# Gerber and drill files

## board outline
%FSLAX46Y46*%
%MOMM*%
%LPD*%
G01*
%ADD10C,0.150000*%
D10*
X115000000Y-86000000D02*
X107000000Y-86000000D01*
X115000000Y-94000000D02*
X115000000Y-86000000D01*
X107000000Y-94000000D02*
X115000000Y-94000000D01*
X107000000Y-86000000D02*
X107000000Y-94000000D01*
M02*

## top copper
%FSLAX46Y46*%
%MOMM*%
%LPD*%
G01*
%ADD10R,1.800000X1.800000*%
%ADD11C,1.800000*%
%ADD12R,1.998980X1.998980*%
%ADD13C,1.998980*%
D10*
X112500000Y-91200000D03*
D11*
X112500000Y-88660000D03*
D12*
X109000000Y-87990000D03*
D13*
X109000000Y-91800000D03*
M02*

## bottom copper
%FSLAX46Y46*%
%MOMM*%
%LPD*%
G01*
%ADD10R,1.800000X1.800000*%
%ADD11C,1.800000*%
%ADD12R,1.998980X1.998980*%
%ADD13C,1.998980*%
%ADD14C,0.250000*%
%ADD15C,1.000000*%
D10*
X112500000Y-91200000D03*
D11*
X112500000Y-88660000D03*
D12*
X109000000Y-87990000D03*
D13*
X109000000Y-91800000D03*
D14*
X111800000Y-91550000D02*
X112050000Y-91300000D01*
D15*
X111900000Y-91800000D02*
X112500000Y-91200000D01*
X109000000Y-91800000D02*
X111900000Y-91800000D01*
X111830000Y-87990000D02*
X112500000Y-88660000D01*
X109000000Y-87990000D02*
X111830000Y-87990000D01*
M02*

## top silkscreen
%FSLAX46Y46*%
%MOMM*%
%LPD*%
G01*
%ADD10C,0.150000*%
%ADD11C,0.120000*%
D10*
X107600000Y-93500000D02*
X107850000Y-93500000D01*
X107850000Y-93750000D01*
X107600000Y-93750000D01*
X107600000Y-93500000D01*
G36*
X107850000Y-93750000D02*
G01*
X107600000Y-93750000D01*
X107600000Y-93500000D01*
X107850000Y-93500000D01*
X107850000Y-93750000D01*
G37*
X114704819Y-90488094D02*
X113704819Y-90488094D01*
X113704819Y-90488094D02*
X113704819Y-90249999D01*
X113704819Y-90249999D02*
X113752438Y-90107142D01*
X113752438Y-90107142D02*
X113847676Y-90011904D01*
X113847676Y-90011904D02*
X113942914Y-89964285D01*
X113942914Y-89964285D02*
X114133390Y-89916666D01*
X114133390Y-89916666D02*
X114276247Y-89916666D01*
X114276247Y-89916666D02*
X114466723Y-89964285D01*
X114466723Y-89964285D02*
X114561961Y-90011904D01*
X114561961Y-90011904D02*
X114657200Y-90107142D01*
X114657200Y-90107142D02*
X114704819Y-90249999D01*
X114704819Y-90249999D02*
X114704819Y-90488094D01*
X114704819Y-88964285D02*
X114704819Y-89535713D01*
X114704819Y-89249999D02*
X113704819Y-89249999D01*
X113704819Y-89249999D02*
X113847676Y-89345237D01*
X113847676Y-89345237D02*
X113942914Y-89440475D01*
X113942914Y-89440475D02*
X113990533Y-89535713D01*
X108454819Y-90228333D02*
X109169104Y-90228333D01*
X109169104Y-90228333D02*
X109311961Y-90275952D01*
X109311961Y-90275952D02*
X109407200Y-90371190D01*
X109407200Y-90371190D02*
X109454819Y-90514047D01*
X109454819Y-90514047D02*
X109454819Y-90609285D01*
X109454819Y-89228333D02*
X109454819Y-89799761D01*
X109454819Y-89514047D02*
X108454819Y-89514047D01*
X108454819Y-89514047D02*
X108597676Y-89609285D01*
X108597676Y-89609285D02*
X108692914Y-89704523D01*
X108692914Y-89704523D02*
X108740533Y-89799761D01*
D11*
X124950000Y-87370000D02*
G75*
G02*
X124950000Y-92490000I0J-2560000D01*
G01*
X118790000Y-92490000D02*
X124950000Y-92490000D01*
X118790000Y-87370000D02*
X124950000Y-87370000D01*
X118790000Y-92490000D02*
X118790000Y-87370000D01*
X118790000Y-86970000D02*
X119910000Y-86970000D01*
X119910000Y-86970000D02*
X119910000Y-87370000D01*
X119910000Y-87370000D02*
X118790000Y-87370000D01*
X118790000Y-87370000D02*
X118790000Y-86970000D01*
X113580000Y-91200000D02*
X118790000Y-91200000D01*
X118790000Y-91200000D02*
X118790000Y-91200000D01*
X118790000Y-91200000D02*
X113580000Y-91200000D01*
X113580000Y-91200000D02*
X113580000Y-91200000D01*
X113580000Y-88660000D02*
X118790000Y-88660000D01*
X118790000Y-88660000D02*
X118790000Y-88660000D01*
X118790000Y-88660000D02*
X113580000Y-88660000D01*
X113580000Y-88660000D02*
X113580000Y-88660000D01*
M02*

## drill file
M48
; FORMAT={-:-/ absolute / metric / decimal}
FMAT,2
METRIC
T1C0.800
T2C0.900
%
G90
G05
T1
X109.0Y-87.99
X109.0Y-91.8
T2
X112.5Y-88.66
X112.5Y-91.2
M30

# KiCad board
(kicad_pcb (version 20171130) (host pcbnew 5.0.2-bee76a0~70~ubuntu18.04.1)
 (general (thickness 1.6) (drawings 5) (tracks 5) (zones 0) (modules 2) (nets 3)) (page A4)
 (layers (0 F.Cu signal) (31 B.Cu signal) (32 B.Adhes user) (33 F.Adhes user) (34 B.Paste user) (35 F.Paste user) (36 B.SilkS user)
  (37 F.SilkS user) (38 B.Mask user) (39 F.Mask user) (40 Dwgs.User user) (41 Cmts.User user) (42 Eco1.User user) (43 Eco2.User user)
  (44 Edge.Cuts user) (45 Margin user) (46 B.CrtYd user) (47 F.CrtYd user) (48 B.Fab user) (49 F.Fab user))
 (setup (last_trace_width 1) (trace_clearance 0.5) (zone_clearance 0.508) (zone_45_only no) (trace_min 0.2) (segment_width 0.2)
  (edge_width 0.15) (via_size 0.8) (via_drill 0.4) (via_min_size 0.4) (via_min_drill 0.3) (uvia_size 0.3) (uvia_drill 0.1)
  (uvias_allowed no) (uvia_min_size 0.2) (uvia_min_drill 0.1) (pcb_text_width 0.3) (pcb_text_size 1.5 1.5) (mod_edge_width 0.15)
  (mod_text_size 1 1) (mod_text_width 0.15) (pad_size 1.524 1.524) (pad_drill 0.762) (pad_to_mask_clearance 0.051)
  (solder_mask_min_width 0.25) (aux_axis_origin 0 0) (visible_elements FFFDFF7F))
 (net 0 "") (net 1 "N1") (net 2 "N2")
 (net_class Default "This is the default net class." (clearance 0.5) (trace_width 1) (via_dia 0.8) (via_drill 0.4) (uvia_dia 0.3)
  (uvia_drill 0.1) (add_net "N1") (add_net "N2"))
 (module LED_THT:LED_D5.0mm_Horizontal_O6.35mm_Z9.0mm (layer F.Cu) (at 112.5 91.2 90)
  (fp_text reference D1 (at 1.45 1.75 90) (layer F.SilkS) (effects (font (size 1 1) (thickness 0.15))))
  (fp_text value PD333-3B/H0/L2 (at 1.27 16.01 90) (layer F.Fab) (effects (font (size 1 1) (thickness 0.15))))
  (fp_arc (start 1.27 12.45) (end -1.29 12.45) (angle -180) (layer F.SilkS) (width 0.12))
  (fp_line (start -1.29 6.29) (end -1.29 12.45) (layer F.SilkS) (width 0.12))
  (fp_line (start 3.83 6.29) (end 3.83 12.45) (layer F.SilkS) (width 0.12))
  (fp_line (start -1.29 6.29) (end 3.83 6.29) (layer F.SilkS) (width 0.12))
  (fp_line (start 4.23 6.29) (end 4.23 7.41) (layer F.SilkS) (width 0.12))
  (fp_line (start 4.23 7.41) (end 3.83 7.41) (layer F.SilkS) (width 0.12))
  (fp_line (start 3.83 7.41) (end 3.83 6.29) (layer F.SilkS) (width 0.12))
  (fp_line (start 3.83 6.29) (end 4.23 6.29) (layer F.SilkS) (width 0.12))
  (fp_line (start 0 1.08) (end 0 6.29) (layer F.SilkS) (width 0.12))
  (fp_line (start 0 6.29) (end 0 6.29) (layer F.SilkS) (width 0.12))
  (fp_line (start 0 6.29) (end 0 1.08) (layer F.SilkS) (width 0.12))
  (fp_line (start 0 1.08) (end 0 1.08) (layer F.SilkS) (width 0.12))
  (fp_line (start 2.54 1.08) (end 2.54 6.29) (layer F.SilkS) (width 0.12))
  (fp_line (start 2.54 6.29) (end 2.54 6.29) (layer F.SilkS) (width 0.12))
  (fp_line (start 2.54 6.29) (end 2.54 1.08) (layer F.SilkS) (width 0.12))
  (fp_line (start 2.54 1.08) (end 2.54 1.08) (layer F.SilkS) (width 0.12))
  (pad 1 thru_hole rect (at 0 0 90) (size 1.8 1.8) (drill 0.9) (layers *.Cu *.Mask) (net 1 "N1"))
  (pad 2 thru_hole circle (at 2.54 0 90) (size 1.8 1.8) (drill 0.9) (layers *.Cu *.Mask) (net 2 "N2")))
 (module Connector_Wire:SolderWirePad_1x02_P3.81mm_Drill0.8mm (layer F.Cu) (at 109 87.99 270)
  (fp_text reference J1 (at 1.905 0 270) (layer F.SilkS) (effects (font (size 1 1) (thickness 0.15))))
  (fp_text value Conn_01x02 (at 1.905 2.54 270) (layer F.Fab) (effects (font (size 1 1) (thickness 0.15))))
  (pad 1 thru_hole rect (at 0 0 270) (size 1.99898 1.99898) (drill 0.8001) (layers *.Cu *.Mask) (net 2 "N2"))
  (pad 2 thru_hole circle (at 3.81 0 270) (size 1.99898 1.99898) (drill 0.8001) (layers *.Cu *.Mask) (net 1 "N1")))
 (gr_poly (pts (xy 107.6 93.5) (xy 107.85 93.5) (xy 107.85 93.75) (xy 107.6 93.75)) (layer F.SilkS) (width 0.15))
 (gr_line (start 115 86) (end 107 86) (layer Edge.Cuts) (width 0.15))
 (gr_line (start 115 94) (end 115 86) (layer Edge.Cuts) (width 0.15))
 (gr_line (start 107 94) (end 115 94) (layer Edge.Cuts) (width 0.15))
 (gr_line (start 107 86) (end 107 94) (layer Edge.Cuts) (width 0.15))
 (segment (start 111.8 91.55) (end 112.05 91.3) (width 0.25) (layer B.Cu) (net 1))
 (segment (start 111.9 91.8) (end 112.5 91.2) (width 1) (layer B.Cu) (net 1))
 (segment (start 109 91.8) (end 111.9 91.8) (width 1) (layer B.Cu) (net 1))
 (segment (start 111.83 87.99) (end 112.5 88.66) (width 1) (layer B.Cu) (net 2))
 (segment (start 109 87.99) (end 111.83 87.99) (width 1) (layer B.Cu) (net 2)))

